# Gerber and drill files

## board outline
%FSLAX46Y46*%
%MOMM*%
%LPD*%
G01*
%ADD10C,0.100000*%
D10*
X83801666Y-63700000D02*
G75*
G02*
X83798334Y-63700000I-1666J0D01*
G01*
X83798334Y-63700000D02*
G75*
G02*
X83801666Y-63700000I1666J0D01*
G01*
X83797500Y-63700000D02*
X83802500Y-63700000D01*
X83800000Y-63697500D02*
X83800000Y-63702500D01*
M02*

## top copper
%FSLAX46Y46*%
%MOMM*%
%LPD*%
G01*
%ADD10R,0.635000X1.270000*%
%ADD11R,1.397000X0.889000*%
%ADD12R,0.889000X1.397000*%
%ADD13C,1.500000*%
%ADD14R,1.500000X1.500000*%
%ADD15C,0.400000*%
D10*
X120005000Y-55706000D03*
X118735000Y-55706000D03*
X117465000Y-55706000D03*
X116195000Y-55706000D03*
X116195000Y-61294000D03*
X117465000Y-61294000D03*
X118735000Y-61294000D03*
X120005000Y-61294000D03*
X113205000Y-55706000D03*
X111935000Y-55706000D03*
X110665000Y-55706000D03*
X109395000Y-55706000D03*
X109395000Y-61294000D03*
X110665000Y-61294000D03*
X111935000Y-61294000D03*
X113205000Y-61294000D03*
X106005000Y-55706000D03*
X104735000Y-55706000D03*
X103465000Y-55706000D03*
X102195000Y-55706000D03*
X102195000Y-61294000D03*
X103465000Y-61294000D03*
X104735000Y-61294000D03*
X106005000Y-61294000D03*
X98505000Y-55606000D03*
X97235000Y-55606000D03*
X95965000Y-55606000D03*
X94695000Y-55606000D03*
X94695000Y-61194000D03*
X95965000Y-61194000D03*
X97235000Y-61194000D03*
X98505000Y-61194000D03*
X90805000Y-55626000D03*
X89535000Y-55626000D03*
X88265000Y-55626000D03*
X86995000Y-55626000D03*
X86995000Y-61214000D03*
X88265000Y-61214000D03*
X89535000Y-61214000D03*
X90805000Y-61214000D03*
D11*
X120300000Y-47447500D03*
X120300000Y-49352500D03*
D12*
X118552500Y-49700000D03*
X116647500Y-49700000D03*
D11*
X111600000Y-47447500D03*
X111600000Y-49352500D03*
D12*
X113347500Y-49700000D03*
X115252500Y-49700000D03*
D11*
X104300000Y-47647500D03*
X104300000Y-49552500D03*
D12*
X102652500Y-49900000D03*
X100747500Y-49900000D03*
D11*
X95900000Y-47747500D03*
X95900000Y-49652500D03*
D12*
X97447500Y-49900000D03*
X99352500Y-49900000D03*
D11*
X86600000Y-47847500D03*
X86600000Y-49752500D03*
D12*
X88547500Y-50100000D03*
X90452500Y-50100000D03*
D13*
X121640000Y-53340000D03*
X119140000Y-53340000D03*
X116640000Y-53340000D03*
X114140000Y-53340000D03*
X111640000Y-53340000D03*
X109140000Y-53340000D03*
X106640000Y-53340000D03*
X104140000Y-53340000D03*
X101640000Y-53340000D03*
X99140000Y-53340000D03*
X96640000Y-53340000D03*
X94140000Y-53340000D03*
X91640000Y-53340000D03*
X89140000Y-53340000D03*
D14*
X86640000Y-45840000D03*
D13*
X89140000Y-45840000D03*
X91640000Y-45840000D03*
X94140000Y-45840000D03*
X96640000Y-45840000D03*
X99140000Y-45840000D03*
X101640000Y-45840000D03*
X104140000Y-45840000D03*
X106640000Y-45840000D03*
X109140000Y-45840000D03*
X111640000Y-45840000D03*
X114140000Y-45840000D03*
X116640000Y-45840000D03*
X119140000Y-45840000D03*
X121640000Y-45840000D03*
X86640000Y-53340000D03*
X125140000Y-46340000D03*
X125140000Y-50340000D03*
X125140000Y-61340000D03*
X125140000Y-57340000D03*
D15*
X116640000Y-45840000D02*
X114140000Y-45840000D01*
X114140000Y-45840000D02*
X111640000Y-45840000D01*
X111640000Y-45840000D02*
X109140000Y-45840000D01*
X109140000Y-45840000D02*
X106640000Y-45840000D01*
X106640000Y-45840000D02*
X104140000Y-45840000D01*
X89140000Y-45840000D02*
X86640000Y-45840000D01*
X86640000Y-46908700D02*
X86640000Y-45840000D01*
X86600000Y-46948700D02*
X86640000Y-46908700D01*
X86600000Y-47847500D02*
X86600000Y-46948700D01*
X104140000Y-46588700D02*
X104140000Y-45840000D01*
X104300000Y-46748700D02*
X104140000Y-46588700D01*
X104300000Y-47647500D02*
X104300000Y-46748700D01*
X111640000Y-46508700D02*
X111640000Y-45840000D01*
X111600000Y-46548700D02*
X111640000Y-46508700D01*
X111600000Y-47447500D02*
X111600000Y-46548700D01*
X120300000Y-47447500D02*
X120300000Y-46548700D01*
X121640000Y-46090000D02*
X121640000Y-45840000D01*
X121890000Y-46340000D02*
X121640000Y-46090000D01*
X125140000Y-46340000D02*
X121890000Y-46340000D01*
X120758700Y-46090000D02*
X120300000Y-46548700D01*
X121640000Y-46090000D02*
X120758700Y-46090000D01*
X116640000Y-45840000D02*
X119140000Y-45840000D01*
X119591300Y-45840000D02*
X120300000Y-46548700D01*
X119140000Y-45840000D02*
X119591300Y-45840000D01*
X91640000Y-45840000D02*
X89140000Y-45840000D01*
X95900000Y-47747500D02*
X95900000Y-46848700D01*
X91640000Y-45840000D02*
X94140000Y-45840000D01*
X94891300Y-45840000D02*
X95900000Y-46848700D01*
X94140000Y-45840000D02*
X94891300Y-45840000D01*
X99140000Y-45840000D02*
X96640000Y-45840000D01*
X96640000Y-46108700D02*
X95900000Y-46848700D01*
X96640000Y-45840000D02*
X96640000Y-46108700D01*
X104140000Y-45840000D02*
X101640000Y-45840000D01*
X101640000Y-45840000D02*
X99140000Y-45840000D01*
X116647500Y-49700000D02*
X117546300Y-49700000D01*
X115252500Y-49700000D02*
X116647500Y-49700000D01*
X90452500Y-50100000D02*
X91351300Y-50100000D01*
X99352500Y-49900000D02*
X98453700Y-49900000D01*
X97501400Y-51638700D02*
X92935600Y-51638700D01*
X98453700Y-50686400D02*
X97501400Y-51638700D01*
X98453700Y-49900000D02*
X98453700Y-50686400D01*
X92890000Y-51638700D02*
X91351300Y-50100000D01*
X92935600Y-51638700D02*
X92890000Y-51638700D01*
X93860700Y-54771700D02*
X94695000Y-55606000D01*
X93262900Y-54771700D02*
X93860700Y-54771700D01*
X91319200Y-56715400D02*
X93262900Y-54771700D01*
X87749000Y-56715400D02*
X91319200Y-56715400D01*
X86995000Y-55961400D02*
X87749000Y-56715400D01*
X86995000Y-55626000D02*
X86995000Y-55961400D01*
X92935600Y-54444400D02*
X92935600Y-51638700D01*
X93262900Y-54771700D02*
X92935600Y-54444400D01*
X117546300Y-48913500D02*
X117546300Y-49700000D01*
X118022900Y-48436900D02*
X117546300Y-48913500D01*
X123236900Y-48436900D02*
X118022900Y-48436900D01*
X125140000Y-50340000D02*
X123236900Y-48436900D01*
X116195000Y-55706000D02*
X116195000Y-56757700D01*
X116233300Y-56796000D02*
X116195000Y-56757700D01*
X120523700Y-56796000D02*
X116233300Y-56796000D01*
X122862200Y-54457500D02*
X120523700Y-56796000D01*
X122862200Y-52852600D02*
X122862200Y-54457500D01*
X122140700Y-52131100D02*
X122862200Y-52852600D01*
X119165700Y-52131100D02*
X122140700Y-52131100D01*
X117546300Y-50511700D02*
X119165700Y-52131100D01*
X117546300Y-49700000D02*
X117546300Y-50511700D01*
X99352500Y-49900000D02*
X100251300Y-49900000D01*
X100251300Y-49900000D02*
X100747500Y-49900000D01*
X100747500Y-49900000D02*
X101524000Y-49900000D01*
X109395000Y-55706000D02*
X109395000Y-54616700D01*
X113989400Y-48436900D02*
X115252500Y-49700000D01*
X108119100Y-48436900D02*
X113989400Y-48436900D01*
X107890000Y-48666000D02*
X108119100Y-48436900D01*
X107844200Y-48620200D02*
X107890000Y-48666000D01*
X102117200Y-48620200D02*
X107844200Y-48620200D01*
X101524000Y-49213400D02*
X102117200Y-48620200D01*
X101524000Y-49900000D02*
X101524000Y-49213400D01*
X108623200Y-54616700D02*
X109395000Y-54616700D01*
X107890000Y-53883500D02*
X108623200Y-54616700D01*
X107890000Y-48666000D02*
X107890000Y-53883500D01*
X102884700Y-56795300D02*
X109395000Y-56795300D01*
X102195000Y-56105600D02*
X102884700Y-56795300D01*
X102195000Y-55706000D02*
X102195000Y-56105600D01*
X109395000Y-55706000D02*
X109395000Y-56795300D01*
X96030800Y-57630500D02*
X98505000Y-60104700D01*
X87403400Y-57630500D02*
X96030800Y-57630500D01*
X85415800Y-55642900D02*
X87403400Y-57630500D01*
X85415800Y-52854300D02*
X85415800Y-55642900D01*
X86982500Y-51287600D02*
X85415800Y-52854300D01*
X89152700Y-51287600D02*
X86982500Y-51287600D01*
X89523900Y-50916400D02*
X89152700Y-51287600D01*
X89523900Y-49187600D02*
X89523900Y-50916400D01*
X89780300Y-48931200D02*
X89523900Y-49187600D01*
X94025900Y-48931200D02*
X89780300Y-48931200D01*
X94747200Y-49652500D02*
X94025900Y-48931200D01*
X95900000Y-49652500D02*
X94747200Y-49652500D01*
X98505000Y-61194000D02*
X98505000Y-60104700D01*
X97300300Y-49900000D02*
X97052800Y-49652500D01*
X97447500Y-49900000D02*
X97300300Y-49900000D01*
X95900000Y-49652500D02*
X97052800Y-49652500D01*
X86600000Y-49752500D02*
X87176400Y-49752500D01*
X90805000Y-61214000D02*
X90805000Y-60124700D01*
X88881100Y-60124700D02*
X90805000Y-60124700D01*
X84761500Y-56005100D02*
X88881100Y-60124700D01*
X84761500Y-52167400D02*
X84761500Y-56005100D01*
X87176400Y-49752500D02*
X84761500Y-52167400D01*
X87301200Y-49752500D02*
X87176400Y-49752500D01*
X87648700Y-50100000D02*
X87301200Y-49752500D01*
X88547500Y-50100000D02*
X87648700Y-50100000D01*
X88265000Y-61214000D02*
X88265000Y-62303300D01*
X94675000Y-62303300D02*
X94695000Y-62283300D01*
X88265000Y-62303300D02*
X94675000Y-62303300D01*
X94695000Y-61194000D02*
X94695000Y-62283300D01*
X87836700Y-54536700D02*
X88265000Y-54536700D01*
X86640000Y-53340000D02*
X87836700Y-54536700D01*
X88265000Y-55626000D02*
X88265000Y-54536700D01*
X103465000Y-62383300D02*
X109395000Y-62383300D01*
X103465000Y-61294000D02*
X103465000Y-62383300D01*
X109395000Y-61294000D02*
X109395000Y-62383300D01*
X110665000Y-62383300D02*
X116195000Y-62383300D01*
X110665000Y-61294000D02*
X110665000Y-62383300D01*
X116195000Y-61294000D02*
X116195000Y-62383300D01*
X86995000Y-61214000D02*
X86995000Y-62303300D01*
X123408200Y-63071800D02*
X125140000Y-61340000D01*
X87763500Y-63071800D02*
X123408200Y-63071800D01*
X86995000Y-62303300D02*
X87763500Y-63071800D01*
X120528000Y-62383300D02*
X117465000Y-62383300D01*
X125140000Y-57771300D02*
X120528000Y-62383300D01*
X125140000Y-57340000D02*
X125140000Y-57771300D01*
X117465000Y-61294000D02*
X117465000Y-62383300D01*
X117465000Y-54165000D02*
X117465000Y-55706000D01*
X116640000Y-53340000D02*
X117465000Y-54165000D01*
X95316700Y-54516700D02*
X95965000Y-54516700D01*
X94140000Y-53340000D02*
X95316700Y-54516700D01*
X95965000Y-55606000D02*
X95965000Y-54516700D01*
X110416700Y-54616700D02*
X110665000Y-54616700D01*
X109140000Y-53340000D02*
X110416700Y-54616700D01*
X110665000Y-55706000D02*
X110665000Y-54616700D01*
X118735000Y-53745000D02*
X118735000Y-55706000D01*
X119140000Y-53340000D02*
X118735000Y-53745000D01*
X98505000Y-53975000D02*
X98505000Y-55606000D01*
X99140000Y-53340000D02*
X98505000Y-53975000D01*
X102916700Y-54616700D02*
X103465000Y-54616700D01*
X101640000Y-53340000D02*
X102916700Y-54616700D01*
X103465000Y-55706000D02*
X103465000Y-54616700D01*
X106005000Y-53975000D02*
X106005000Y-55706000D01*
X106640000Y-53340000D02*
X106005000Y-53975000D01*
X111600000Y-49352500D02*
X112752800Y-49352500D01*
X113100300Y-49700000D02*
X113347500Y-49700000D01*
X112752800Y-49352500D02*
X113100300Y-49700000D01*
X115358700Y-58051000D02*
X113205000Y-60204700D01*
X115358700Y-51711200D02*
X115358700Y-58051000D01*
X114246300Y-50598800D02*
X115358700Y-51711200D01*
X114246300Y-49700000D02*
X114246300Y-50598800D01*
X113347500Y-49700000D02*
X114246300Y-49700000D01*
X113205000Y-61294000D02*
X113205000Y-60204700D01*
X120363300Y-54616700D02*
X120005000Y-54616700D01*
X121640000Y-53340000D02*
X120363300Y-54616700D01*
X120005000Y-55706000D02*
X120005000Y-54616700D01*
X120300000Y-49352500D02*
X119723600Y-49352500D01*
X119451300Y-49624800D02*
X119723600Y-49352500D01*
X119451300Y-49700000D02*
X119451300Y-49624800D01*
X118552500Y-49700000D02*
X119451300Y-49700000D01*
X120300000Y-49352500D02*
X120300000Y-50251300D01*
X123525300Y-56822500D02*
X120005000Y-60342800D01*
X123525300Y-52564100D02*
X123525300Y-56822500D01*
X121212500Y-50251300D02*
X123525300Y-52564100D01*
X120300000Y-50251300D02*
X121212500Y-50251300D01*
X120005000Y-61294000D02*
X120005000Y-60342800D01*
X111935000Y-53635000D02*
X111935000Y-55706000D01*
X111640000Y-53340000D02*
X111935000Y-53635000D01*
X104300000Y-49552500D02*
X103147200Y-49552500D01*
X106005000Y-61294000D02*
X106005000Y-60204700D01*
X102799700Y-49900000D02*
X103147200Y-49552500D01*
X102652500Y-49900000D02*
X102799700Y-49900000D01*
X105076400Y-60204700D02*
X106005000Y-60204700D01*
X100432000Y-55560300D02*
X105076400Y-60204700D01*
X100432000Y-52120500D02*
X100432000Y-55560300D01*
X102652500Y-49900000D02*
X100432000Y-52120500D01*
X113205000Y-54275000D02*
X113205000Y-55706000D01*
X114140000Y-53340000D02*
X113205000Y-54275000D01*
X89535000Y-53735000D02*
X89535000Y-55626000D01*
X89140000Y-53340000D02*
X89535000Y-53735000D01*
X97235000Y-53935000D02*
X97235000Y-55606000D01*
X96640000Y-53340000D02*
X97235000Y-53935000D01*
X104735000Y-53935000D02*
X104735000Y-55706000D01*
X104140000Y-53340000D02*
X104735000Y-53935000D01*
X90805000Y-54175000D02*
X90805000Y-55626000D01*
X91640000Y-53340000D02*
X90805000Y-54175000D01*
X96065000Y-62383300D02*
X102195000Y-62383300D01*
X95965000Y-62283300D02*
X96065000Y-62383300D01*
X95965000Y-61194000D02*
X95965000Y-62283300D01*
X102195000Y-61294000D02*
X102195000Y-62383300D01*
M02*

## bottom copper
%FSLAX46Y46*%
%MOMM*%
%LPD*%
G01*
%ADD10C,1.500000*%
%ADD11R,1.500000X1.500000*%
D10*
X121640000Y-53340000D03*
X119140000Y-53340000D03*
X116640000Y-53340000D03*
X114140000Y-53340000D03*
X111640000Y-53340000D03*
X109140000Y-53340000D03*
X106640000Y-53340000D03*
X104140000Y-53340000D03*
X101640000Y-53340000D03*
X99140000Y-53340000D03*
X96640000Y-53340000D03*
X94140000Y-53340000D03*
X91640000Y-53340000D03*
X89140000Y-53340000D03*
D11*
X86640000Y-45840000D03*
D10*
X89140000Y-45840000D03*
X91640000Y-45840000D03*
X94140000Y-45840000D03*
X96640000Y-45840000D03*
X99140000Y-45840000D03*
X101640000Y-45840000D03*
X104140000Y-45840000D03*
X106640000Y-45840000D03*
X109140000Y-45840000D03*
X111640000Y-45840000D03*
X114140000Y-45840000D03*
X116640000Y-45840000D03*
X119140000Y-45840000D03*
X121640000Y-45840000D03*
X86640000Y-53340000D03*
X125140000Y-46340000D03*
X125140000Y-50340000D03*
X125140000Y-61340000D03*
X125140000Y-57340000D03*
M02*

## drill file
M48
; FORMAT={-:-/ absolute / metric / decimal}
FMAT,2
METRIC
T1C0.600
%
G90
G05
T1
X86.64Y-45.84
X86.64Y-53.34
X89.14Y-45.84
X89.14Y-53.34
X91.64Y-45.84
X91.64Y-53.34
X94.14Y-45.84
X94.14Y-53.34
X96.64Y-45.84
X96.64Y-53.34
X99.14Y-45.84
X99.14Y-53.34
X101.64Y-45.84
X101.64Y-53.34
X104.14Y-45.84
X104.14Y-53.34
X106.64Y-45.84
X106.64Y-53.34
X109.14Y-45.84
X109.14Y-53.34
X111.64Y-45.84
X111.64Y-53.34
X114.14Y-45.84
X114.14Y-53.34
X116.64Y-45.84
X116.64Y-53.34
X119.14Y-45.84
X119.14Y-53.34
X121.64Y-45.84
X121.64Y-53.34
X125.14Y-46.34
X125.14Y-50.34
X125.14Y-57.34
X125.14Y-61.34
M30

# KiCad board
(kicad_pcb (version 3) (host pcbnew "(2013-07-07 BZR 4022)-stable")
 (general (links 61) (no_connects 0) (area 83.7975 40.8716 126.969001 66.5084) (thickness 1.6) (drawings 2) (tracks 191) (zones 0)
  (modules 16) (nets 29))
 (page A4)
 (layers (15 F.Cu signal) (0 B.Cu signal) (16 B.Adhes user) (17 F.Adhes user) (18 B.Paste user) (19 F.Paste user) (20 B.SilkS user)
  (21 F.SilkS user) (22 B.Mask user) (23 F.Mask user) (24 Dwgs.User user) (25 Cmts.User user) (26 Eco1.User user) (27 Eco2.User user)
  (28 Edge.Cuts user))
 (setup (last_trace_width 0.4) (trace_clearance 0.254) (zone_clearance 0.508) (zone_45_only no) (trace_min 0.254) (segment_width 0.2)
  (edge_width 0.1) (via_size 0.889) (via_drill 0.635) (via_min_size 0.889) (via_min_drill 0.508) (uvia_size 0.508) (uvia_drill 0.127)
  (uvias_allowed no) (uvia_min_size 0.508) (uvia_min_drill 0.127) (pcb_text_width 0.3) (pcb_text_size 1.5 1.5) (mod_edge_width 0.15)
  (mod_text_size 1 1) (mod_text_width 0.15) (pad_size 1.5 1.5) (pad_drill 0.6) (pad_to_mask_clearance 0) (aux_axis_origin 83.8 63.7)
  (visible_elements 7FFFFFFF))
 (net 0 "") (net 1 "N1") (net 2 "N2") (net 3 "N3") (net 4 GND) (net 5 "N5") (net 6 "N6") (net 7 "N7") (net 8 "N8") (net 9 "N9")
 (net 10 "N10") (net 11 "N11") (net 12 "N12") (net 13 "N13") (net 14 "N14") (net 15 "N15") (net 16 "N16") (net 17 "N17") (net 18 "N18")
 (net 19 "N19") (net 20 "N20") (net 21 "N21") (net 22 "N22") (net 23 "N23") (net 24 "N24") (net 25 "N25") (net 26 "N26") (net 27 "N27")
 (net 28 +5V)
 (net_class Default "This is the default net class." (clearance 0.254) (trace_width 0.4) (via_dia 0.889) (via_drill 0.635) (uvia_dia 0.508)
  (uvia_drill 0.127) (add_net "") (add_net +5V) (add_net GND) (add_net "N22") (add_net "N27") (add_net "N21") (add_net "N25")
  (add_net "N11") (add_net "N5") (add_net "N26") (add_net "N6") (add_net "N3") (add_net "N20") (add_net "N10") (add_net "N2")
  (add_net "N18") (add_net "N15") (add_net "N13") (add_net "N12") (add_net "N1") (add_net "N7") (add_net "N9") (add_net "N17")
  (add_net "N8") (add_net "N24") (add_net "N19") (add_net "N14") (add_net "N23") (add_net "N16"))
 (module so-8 (layer F.Cu) (at 118.1 58.5 180)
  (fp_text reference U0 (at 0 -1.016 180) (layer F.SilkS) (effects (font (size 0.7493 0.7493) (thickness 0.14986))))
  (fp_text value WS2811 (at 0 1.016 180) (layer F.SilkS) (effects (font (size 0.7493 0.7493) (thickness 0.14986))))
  (pad 1 smd rect (at -1.905 2.794 180) (size 0.635 1.27) (layers F.Cu F.Paste F.Mask) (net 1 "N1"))
  (pad 2 smd rect (at -0.635 2.794 180) (size 0.635 1.27) (layers F.Cu F.Paste F.Mask) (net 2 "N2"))
  (pad 3 smd rect (at 0.635 2.794 180) (size 0.635 1.27) (layers F.Cu F.Paste F.Mask) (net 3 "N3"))
  (pad 4 smd rect (at 1.905 2.794 180) (size 0.635 1.27) (layers F.Cu F.Paste F.Mask) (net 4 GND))
  (pad 5 smd rect (at 1.905 -2.794 180) (size 0.635 1.27) (layers F.Cu F.Paste F.Mask) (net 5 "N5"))
  (pad 6 smd rect (at 0.635 -2.794 180) (size 0.635 1.27) (layers F.Cu F.Paste F.Mask) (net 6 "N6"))
  (pad 7 smd rect (at -0.635 -2.794 180) (size 0.635 1.27) (layers F.Cu F.Paste F.Mask))
  (pad 8 smd rect (at -1.905 -2.794 180) (size 0.635 1.27) (layers F.Cu F.Paste F.Mask) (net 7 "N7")))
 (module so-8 (layer F.Cu) (at 111.3 58.5 180)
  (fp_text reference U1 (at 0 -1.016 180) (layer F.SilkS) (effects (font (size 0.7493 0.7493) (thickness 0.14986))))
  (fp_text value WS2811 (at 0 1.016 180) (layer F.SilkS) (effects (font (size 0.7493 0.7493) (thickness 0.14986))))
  (pad 1 smd rect (at -1.905 2.794 180) (size 0.635 1.27) (layers F.Cu F.Paste F.Mask) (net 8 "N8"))
  (pad 2 smd rect (at -0.635 2.794 180) (size 0.635 1.27) (layers F.Cu F.Paste F.Mask) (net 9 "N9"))
  (pad 3 smd rect (at 0.635 2.794 180) (size 0.635 1.27) (layers F.Cu F.Paste F.Mask) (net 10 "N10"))
  (pad 4 smd rect (at 1.905 2.794 180) (size 0.635 1.27) (layers F.Cu F.Paste F.Mask) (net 4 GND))
  (pad 5 smd rect (at 1.905 -2.794 180) (size 0.635 1.27) (layers F.Cu F.Paste F.Mask) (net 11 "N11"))
  (pad 6 smd rect (at 0.635 -2.794 180) (size 0.635 1.27) (layers F.Cu F.Paste F.Mask) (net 5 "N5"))
  (pad 7 smd rect (at -0.635 -2.794 180) (size 0.635 1.27) (layers F.Cu F.Paste F.Mask))
  (pad 8 smd rect (at -1.905 -2.794 180) (size 0.635 1.27) (layers F.Cu F.Paste F.Mask) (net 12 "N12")))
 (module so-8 (layer F.Cu) (at 104.1 58.5 180)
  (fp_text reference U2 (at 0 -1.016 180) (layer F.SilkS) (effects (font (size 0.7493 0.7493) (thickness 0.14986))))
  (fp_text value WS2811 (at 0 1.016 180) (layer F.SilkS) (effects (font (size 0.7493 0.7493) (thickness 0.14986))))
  (pad 1 smd rect (at -1.905 2.794 180) (size 0.635 1.27) (layers F.Cu F.Paste F.Mask) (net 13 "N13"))
  (pad 2 smd rect (at -0.635 2.794 180) (size 0.635 1.27) (layers F.Cu F.Paste F.Mask) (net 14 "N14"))
  (pad 3 smd rect (at 0.635 2.794 180) (size 0.635 1.27) (layers F.Cu F.Paste F.Mask) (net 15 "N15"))
  (pad 4 smd rect (at 1.905 2.794 180) (size 0.635 1.27) (layers F.Cu F.Paste F.Mask) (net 4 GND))
  (pad 5 smd rect (at 1.905 -2.794 180) (size 0.635 1.27) (layers F.Cu F.Paste F.Mask) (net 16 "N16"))
  (pad 6 smd rect (at 0.635 -2.794 180) (size 0.635 1.27) (layers F.Cu F.Paste F.Mask) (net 11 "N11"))
  (pad 7 smd rect (at -0.635 -2.794 180) (size 0.635 1.27) (layers F.Cu F.Paste F.Mask))
  (pad 8 smd rect (at -1.905 -2.794 180) (size 0.635 1.27) (layers F.Cu F.Paste F.Mask) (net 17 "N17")))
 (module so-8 (layer F.Cu) (at 96.6 58.4 180)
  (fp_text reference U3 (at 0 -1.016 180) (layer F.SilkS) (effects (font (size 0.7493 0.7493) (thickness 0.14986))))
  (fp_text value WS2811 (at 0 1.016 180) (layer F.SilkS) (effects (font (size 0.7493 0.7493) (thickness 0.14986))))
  (pad 1 smd rect (at -1.905 2.794 180) (size 0.635 1.27) (layers F.Cu F.Paste F.Mask) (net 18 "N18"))
  (pad 2 smd rect (at -0.635 2.794 180) (size 0.635 1.27) (layers F.Cu F.Paste F.Mask) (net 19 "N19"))
  (pad 3 smd rect (at 0.635 2.794 180) (size 0.635 1.27) (layers F.Cu F.Paste F.Mask) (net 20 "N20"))
  (pad 4 smd rect (at 1.905 2.794 180) (size 0.635 1.27) (layers F.Cu F.Paste F.Mask) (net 4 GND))
  (pad 5 smd rect (at 1.905 -2.794 180) (size 0.635 1.27) (layers F.Cu F.Paste F.Mask) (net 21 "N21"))
  (pad 6 smd rect (at 0.635 -2.794 180) (size 0.635 1.27) (layers F.Cu F.Paste F.Mask) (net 16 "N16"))
  (pad 7 smd rect (at -0.635 -2.794 180) (size 0.635 1.27) (layers F.Cu F.Paste F.Mask))
  (pad 8 smd rect (at -1.905 -2.794 180) (size 0.635 1.27) (layers F.Cu F.Paste F.Mask) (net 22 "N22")))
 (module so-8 (layer F.Cu) (at 88.9 58.42 180)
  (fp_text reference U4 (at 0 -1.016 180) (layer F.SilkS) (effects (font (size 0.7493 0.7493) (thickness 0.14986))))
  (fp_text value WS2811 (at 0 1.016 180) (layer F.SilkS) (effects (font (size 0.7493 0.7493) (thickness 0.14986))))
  (pad 1 smd rect (at -1.905 2.794 180) (size 0.635 1.27) (layers F.Cu F.Paste F.Mask) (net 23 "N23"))
  (pad 2 smd rect (at -0.635 2.794 180) (size 0.635 1.27) (layers F.Cu F.Paste F.Mask) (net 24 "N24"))
  (pad 3 smd rect (at 0.635 2.794 180) (size 0.635 1.27) (layers F.Cu F.Paste F.Mask) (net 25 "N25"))
  (pad 4 smd rect (at 1.905 2.794 180) (size 0.635 1.27) (layers F.Cu F.Paste F.Mask) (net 4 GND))
  (pad 5 smd rect (at 1.905 -2.794 180) (size 0.635 1.27) (layers F.Cu F.Paste F.Mask) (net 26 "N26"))
  (pad 6 smd rect (at 0.635 -2.794 180) (size 0.635 1.27) (layers F.Cu F.Paste F.Mask) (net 21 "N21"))
  (pad 7 smd rect (at -0.635 -2.794 180) (size 0.635 1.27) (layers F.Cu F.Paste F.Mask))
  (pad 8 smd rect (at -1.905 -2.794 180) (size 0.635 1.27) (layers F.Cu F.Paste F.Mask) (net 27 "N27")))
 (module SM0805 (layer F.Cu) (at 120.3 48.4 270)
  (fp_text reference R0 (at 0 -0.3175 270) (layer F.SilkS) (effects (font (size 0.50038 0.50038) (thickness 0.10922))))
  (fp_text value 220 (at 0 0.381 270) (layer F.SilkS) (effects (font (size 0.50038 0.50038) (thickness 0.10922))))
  (pad 1 smd rect (at -0.9525 0 270) (size 0.889 1.397) (layers F.Cu F.Paste F.Mask) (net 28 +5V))
  (pad 2 smd rect (at 0.9525 0 270) (size 0.889 1.397) (layers F.Cu F.Paste F.Mask) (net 7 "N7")))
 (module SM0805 (layer F.Cu) (at 117.6 49.7 180)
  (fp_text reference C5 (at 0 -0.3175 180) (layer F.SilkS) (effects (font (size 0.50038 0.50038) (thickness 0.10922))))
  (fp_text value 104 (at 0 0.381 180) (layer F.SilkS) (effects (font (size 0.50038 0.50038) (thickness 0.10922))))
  (pad 1 smd rect (at -0.9525 0 180) (size 0.889 1.397) (layers F.Cu F.Paste F.Mask) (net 7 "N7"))
  (pad 2 smd rect (at 0.9525 0 180) (size 0.889 1.397) (layers F.Cu F.Paste F.Mask) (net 4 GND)))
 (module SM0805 (layer F.Cu) (at 111.6 48.4 270)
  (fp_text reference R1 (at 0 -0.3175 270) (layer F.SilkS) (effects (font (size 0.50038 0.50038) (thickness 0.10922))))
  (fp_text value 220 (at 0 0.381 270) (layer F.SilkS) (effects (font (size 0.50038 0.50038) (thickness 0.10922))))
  (pad 1 smd rect (at -0.9525 0 270) (size 0.889 1.397) (layers F.Cu F.Paste F.Mask) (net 28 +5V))
  (pad 2 smd rect (at 0.9525 0 270) (size 0.889 1.397) (layers F.Cu F.Paste F.Mask) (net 12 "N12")))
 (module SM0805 (layer F.Cu) (at 114.3 49.7)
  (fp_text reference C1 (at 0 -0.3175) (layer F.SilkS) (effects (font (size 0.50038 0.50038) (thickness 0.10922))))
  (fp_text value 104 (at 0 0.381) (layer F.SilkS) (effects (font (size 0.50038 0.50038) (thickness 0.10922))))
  (pad 1 smd rect (at -0.9525 0) (size 0.889 1.397) (layers F.Cu F.Paste F.Mask) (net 12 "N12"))
  (pad 2 smd rect (at 0.9525 0) (size 0.889 1.397) (layers F.Cu F.Paste F.Mask) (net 4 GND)))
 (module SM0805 (layer F.Cu) (at 104.3 48.6 270)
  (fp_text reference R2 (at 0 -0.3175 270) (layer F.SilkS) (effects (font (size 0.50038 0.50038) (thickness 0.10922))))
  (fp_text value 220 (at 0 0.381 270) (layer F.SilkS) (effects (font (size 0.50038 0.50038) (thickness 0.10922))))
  (pad 1 smd rect (at -0.9525 0 270) (size 0.889 1.397) (layers F.Cu F.Paste F.Mask) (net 28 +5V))
  (pad 2 smd rect (at 0.9525 0 270) (size 0.889 1.397) (layers F.Cu F.Paste F.Mask) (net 17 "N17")))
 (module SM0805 (layer F.Cu) (at 101.7 49.9 180)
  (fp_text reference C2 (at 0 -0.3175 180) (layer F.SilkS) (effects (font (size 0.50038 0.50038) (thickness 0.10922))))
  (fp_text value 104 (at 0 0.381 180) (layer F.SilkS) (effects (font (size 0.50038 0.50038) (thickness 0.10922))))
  (pad 1 smd rect (at -0.9525 0 180) (size 0.889 1.397) (layers F.Cu F.Paste F.Mask) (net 17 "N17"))
  (pad 2 smd rect (at 0.9525 0 180) (size 0.889 1.397) (layers F.Cu F.Paste F.Mask) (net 4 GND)))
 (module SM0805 (layer F.Cu) (at 95.9 48.7 270)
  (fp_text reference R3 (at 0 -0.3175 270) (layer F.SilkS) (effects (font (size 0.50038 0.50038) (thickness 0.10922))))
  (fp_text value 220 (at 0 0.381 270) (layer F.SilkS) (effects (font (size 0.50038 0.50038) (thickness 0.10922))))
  (pad 1 smd rect (at -0.9525 0 270) (size 0.889 1.397) (layers F.Cu F.Paste F.Mask) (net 28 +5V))
  (pad 2 smd rect (at 0.9525 0 270) (size 0.889 1.397) (layers F.Cu F.Paste F.Mask) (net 22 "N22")))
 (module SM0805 (layer F.Cu) (at 98.4 49.9)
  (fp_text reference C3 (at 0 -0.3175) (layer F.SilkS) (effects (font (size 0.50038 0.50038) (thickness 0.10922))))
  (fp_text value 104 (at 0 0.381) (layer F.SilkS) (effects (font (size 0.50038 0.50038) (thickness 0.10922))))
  (pad 1 smd rect (at -0.9525 0) (size 0.889 1.397) (layers F.Cu F.Paste F.Mask) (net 22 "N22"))
  (pad 2 smd rect (at 0.9525 0) (size 0.889 1.397) (layers F.Cu F.Paste F.Mask) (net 4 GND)))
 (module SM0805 (layer F.Cu) (at 86.6 48.8 270)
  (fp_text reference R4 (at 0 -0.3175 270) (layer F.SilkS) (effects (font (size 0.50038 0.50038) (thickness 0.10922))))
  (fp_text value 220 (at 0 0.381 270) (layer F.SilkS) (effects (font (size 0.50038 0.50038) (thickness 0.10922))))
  (pad 1 smd rect (at -0.9525 0 270) (size 0.889 1.397) (layers F.Cu F.Paste F.Mask) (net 28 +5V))
  (pad 2 smd rect (at 0.9525 0 270) (size 0.889 1.397) (layers F.Cu F.Paste F.Mask) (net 27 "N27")))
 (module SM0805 (layer F.Cu) (at 89.5 50.1)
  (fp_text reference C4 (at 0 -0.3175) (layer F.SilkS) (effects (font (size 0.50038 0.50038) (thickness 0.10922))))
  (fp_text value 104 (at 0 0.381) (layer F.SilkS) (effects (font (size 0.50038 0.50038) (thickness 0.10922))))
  (pad 1 smd rect (at -0.9525 0) (size 0.889 1.397) (layers F.Cu F.Paste F.Mask) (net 27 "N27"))
  (pad 2 smd rect (at 0.9525 0) (size 0.889 1.397) (layers F.Cu F.Paste F.Mask) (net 4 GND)))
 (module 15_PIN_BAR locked (layer F.Cu) (at 104.14 53.34)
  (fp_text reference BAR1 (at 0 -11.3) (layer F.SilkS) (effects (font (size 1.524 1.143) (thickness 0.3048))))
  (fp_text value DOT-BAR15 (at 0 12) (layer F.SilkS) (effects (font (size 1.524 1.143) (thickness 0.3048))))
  (pad 16 thru_hole circle (at 17.5 0) (size 1.5 1.5) (drill 0.6) (layers *.Cu *.Mask F.SilkS) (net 1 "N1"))
  (pad 17 thru_hole circle (at 15 0) (size 1.5 1.5) (drill 0.6) (layers *.Cu *.Mask F.SilkS) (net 2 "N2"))
  (pad 18 thru_hole circle (at 12.5 0) (size 1.5 1.5) (drill 0.6) (layers *.Cu *.Mask F.SilkS) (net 3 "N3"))
  (pad 19 thru_hole circle (at 10 0) (size 1.5 1.5) (drill 0.6) (layers *.Cu *.Mask F.SilkS) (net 8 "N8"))
  (pad 20 thru_hole circle (at 7.5 0) (size 1.5 1.5) (drill 0.6) (layers *.Cu *.Mask F.SilkS) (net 9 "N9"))
  (pad 21 thru_hole circle (at 5 0) (size 1.5 1.5) (drill 0.6) (layers *.Cu *.Mask F.SilkS) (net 10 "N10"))
  (pad 22 thru_hole circle (at 2.5 0) (size 1.5 1.5) (drill 0.6) (layers *.Cu *.Mask F.SilkS) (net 13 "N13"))
  (pad 23 thru_hole circle (at 0 0) (size 1.5 1.5) (drill 0.6) (layers *.Cu *.Mask F.SilkS) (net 14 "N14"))
  (pad 24 thru_hole circle (at -2.5 0) (size 1.5 1.5) (drill 0.6) (layers *.Cu *.Mask F.SilkS) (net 15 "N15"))
  (pad 25 thru_hole circle (at -5 0) (size 1.5 1.5) (drill 0.6) (layers *.Cu *.Mask F.SilkS) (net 18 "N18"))
  (pad 26 thru_hole circle (at -7.5 0) (size 1.5 1.5) (drill 0.6) (layers *.Cu *.Mask F.SilkS) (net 19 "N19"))
  (pad 27 thru_hole circle (at -10 0) (size 1.5 1.5) (drill 0.6) (layers *.Cu *.Mask F.SilkS) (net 20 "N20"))
  (pad 28 thru_hole circle (at -12.5 0) (size 1.5 1.5) (drill 0.6) (layers *.Cu *.Mask F.SilkS) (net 23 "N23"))
  (pad 29 thru_hole circle (at -15 0) (size 1.5 1.5) (drill 0.6) (layers *.Cu *.Mask F.SilkS) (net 24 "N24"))
  (pad 1 thru_hole rect (at -17.5 -7.5) (size 1.5 1.5) (drill 0.6) (layers *.Cu *.Mask F.SilkS) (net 28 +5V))
  (pad 2 thru_hole circle (at -15 -7.5) (size 1.5 1.5) (drill 0.6) (layers *.Cu *.Mask F.SilkS) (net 28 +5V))
  (pad 3 thru_hole circle (at -12.5 -7.5) (size 1.5 1.5) (drill 0.6) (layers *.Cu *.Mask F.SilkS) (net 28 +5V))
  (pad 4 thru_hole circle (at -10 -7.5) (size 1.5 1.5) (drill 0.6) (layers *.Cu *.Mask F.SilkS) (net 28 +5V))
  (pad 5 thru_hole circle (at -7.5 -7.5) (size 1.5 1.5) (drill 0.6) (layers *.Cu *.Mask F.SilkS) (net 28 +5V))
  (pad 6 thru_hole circle (at -5 -7.5) (size 1.5 1.5) (drill 0.6) (layers *.Cu *.Mask F.SilkS) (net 28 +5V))
  (pad 7 thru_hole circle (at -2.5 -7.5) (size 1.5 1.5) (drill 0.6) (layers *.Cu *.Mask F.SilkS) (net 28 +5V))
  (pad 8 thru_hole circle (at 0 -7.5) (size 1.5 1.5) (drill 0.6) (layers *.Cu *.Mask F.SilkS) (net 28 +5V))
  (pad 9 thru_hole circle (at 2.5 -7.5) (size 1.5 1.5) (drill 0.6) (layers *.Cu *.Mask F.SilkS) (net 28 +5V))
  (pad 10 thru_hole circle (at 5 -7.5) (size 1.5 1.5) (drill 0.6) (layers *.Cu *.Mask F.SilkS) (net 28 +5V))
  (pad 11 thru_hole circle (at 7.5 -7.5) (size 1.5 1.5) (drill 0.6) (layers *.Cu *.Mask F.SilkS) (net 28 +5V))
  (pad 12 thru_hole circle (at 10 -7.5) (size 1.5 1.5) (drill 0.6) (layers *.Cu *.Mask F.SilkS) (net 28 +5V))
  (pad 13 thru_hole circle (at 12.5 -7.5) (size 1.5 1.5) (drill 0.6) (layers *.Cu *.Mask F.SilkS) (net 28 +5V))
  (pad 14 thru_hole circle (at 15 -7.5) (size 1.5 1.5) (drill 0.6) (layers *.Cu *.Mask F.SilkS) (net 28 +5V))
  (pad 15 thru_hole circle (at 17.5 -7.5) (size 1.5 1.5) (drill 0.6) (layers *.Cu *.Mask F.SilkS) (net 28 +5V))
  (pad 30 thru_hole circle (at -17.5 0) (size 1.5 1.5) (drill 0.6) (layers *.Cu *.Mask F.SilkS) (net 25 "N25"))
  (pad 31 thru_hole circle (at 21 -7) (size 1.5 1.5) (drill 0.6) (layers *.Cu *.Mask F.SilkS) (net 28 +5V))
  (pad 32 thru_hole circle (at 21 -3) (size 1.5 1.5) (drill 0.6) (layers *.Cu *.Mask F.SilkS) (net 4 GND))
  (pad 33 thru_hole circle (at 21 8) (size 1.5 1.5) (drill 0.6) (layers *.Cu *.Mask F.SilkS) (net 26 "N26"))
  (pad 34 thru_hole circle (at 21 4) (size 1.5 1.5) (drill 0.6) (layers *.Cu *.Mask F.SilkS) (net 6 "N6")))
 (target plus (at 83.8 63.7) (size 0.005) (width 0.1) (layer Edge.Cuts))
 (segment (start 116.64 45.84) (end 114.14 45.84) (width 0.4) (layer F.Cu) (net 28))
 (segment (start 114.14 45.84) (end 111.64 45.84) (width 0.4) (layer F.Cu) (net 28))
 (segment (start 111.64 45.84) (end 109.14 45.84) (width 0.4) (layer F.Cu) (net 28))
 (segment (start 109.14 45.84) (end 106.64 45.84) (width 0.4) (layer F.Cu) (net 28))
 (segment (start 106.64 45.84) (end 104.14 45.84) (width 0.4) (layer F.Cu) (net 28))
 (segment (start 89.14 45.84) (end 86.64 45.84) (width 0.4) (layer F.Cu) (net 28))
 (segment (start 86.64 46.9087) (end 86.64 45.84) (width 0.4) (layer F.Cu) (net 28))
 (segment (start 86.6 46.9487) (end 86.64 46.9087) (width 0.4) (layer F.Cu) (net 28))
 (segment (start 86.6 47.8475) (end 86.6 46.9487) (width 0.4) (layer F.Cu) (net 28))
 (segment (start 104.14 46.5887) (end 104.14 45.84) (width 0.4) (layer F.Cu) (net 28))
 (segment (start 104.3 46.7487) (end 104.14 46.5887) (width 0.4) (layer F.Cu) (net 28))
 (segment (start 104.3 47.6475) (end 104.3 46.7487) (width 0.4) (layer F.Cu) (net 28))
 (segment (start 111.64 46.5087) (end 111.64 45.84) (width 0.4) (layer F.Cu) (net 28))
 (segment (start 111.6 46.5487) (end 111.64 46.5087) (width 0.4) (layer F.Cu) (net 28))
 (segment (start 111.6 47.4475) (end 111.6 46.5487) (width 0.4) (layer F.Cu) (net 28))
 (segment (start 120.3 47.4475) (end 120.3 46.5487) (width 0.4) (layer F.Cu) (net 28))
 (segment (start 121.64 46.09) (end 121.64 45.84) (width 0.4) (layer F.Cu) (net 28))
 (segment (start 121.89 46.34) (end 121.64 46.09) (width 0.4) (layer F.Cu) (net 28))
 (segment (start 125.14 46.34) (end 121.89 46.34) (width 0.4) (layer F.Cu) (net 28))
 (segment (start 120.7587 46.09) (end 120.3 46.5487) (width 0.4) (layer F.Cu) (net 28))
 (segment (start 121.64 46.09) (end 120.7587 46.09) (width 0.4) (layer F.Cu) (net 28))
 (segment (start 116.64 45.84) (end 119.14 45.84) (width 0.4) (layer F.Cu) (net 28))
 (segment (start 119.5913 45.84) (end 120.3 46.5487) (width 0.4) (layer F.Cu) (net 28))
 (segment (start 119.14 45.84) (end 119.5913 45.84) (width 0.4) (layer F.Cu) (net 28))
 (segment (start 91.64 45.84) (end 89.14 45.84) (width 0.4) (layer F.Cu) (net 28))
 (segment (start 95.9 47.7475) (end 95.9 46.8487) (width 0.4) (layer F.Cu) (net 28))
 (segment (start 91.64 45.84) (end 94.14 45.84) (width 0.4) (layer F.Cu) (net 28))
 (segment (start 94.8913 45.84) (end 95.9 46.8487) (width 0.4) (layer F.Cu) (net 28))
 (segment (start 94.14 45.84) (end 94.8913 45.84) (width 0.4) (layer F.Cu) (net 28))
 (segment (start 99.14 45.84) (end 96.64 45.84) (width 0.4) (layer F.Cu) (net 28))
 (segment (start 96.64 46.1087) (end 95.9 46.8487) (width 0.4) (layer F.Cu) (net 28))
 (segment (start 96.64 45.84) (end 96.64 46.1087) (width 0.4) (layer F.Cu) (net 28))
 (segment (start 104.14 45.84) (end 101.64 45.84) (width 0.4) (layer F.Cu) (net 28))
 (segment (start 101.64 45.84) (end 99.14 45.84) (width 0.4) (layer F.Cu) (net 28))
 (segment (start 116.6475 49.7) (end 117.5463 49.7) (width 0.4) (layer F.Cu) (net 4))
 (segment (start 115.2525 49.7) (end 116.6475 49.7) (width 0.4) (layer F.Cu) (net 4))
 (segment (start 90.4525 50.1) (end 91.3513 50.1) (width 0.4) (layer F.Cu) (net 4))
 (segment (start 99.3525 49.9) (end 98.4537 49.9) (width 0.4) (layer F.Cu) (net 4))
 (segment (start 97.5014 51.6387) (end 92.9356 51.6387) (width 0.4) (layer F.Cu) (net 4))
 (segment (start 98.4537 50.6864) (end 97.5014 51.6387) (width 0.4) (layer F.Cu) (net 4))
 (segment (start 98.4537 49.9) (end 98.4537 50.6864) (width 0.4) (layer F.Cu) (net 4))
 (segment (start 92.89 51.6387) (end 91.3513 50.1) (width 0.4) (layer F.Cu) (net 4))
 (segment (start 92.9356 51.6387) (end 92.89 51.6387) (width 0.4) (layer F.Cu) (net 4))
 (segment (start 93.8607 54.7717) (end 94.695 55.606) (width 0.4) (layer F.Cu) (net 4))
 (segment (start 93.2629 54.7717) (end 93.8607 54.7717) (width 0.4) (layer F.Cu) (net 4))
 (segment (start 91.3192 56.7154) (end 93.2629 54.7717) (width 0.4) (layer F.Cu) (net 4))
 (segment (start 87.749 56.7154) (end 91.3192 56.7154) (width 0.4) (layer F.Cu) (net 4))
 (segment (start 86.995 55.9614) (end 87.749 56.7154) (width 0.4) (layer F.Cu) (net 4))
 (segment (start 86.995 55.626) (end 86.995 55.9614) (width 0.4) (layer F.Cu) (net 4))
 (segment (start 92.9356 54.4444) (end 92.9356 51.6387) (width 0.4) (layer F.Cu) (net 4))
 (segment (start 93.2629 54.7717) (end 92.9356 54.4444) (width 0.4) (layer F.Cu) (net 4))
 (segment (start 117.5463 48.9135) (end 117.5463 49.7) (width 0.4) (layer F.Cu) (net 4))
 (segment (start 118.0229 48.4369) (end 117.5463 48.9135) (width 0.4) (layer F.Cu) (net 4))
 (segment (start 123.2369 48.4369) (end 118.0229 48.4369) (width 0.4) (layer F.Cu) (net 4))
 (segment (start 125.14 50.34) (end 123.2369 48.4369) (width 0.4) (layer F.Cu) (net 4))
 (segment (start 116.195 55.706) (end 116.195 56.7577) (width 0.4) (layer F.Cu) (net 4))
 (segment (start 116.2333 56.796) (end 116.195 56.7577) (width 0.4) (layer F.Cu) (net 4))
 (segment (start 120.5237 56.796) (end 116.2333 56.796) (width 0.4) (layer F.Cu) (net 4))
 (segment (start 122.8622 54.4575) (end 120.5237 56.796) (width 0.4) (layer F.Cu) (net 4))
 (segment (start 122.8622 52.8526) (end 122.8622 54.4575) (width 0.4) (layer F.Cu) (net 4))
 (segment (start 122.1407 52.1311) (end 122.8622 52.8526) (width 0.4) (layer F.Cu) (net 4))
 (segment (start 119.1657 52.1311) (end 122.1407 52.1311) (width 0.4) (layer F.Cu) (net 4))
 (segment (start 117.5463 50.5117) (end 119.1657 52.1311) (width 0.4) (layer F.Cu) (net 4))
 (segment (start 117.5463 49.7) (end 117.5463 50.5117) (width 0.4) (layer F.Cu) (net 4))
 (segment (start 99.3525 49.9) (end 100.2513 49.9) (width 0.4) (layer F.Cu) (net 4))
 (segment (start 100.2513 49.9) (end 100.7475 49.9) (width 0.4) (layer F.Cu) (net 4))
 (segment (start 100.7475 49.9) (end 101.524 49.9) (width 0.4) (layer F.Cu) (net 4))
 (segment (start 109.395 55.706) (end 109.395 54.6167) (width 0.4) (layer F.Cu) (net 4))
 (segment (start 113.9894 48.4369) (end 115.2525 49.7) (width 0.4) (layer F.Cu) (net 4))
 (segment (start 108.1191 48.4369) (end 113.9894 48.4369) (width 0.4) (layer F.Cu) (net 4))
 (segment (start 107.89 48.666) (end 108.1191 48.4369) (width 0.4) (layer F.Cu) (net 4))
 (segment (start 107.8442 48.6202) (end 107.89 48.666) (width 0.4) (layer F.Cu) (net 4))
 (segment (start 102.1172 48.6202) (end 107.8442 48.6202) (width 0.4) (layer F.Cu) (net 4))
 (segment (start 101.524 49.2134) (end 102.1172 48.6202) (width 0.4) (layer F.Cu) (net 4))
 (segment (start 101.524 49.9) (end 101.524 49.2134) (width 0.4) (layer F.Cu) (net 4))
 (segment (start 108.6232 54.6167) (end 109.395 54.6167) (width 0.4) (layer F.Cu) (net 4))
 (segment (start 107.89 53.8835) (end 108.6232 54.6167) (width 0.4) (layer F.Cu) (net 4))
 (segment (start 107.89 48.666) (end 107.89 53.8835) (width 0.4) (layer F.Cu) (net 4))
 (segment (start 102.8847 56.7953) (end 109.395 56.7953) (width 0.4) (layer F.Cu) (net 4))
 (segment (start 102.195 56.1056) (end 102.8847 56.7953) (width 0.4) (layer F.Cu) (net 4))
 (segment (start 102.195 55.706) (end 102.195 56.1056) (width 0.4) (layer F.Cu) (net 4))
 (segment (start 109.395 55.706) (end 109.395 56.7953) (width 0.4) (layer F.Cu) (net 4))
 (segment (start 96.0308 57.6305) (end 98.505 60.1047) (width 0.4) (layer F.Cu) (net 22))
 (segment (start 87.4034 57.6305) (end 96.0308 57.6305) (width 0.4) (layer F.Cu) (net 22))
 (segment (start 85.4158 55.6429) (end 87.4034 57.6305) (width 0.4) (layer F.Cu) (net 22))
 (segment (start 85.4158 52.8543) (end 85.4158 55.6429) (width 0.4) (layer F.Cu) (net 22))
 (segment (start 86.9825 51.2876) (end 85.4158 52.8543) (width 0.4) (layer F.Cu) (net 22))
 (segment (start 89.1527 51.2876) (end 86.9825 51.2876) (width 0.4) (layer F.Cu) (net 22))
 (segment (start 89.5239 50.9164) (end 89.1527 51.2876) (width 0.4) (layer F.Cu) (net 22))
 (segment (start 89.5239 49.1876) (end 89.5239 50.9164) (width 0.4) (layer F.Cu) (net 22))
 (segment (start 89.7803 48.9312) (end 89.5239 49.1876) (width 0.4) (layer F.Cu) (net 22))
 (segment (start 94.0259 48.9312) (end 89.7803 48.9312) (width 0.4) (layer F.Cu) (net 22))
 (segment (start 94.7472 49.6525) (end 94.0259 48.9312) (width 0.4) (layer F.Cu) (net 22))
 (segment (start 95.9 49.6525) (end 94.7472 49.6525) (width 0.4) (layer F.Cu) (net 22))
 (segment (start 98.505 61.194) (end 98.505 60.1047) (width 0.4) (layer F.Cu) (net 22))
 (segment (start 97.3003 49.9) (end 97.0528 49.6525) (width 0.4) (layer F.Cu) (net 22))
 (segment (start 97.4475 49.9) (end 97.3003 49.9) (width 0.4) (layer F.Cu) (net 22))
 (segment (start 95.9 49.6525) (end 97.0528 49.6525) (width 0.4) (layer F.Cu) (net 22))
 (segment (start 86.6 49.7525) (end 87.1764 49.7525) (width 0.4) (layer F.Cu) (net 27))
 (segment (start 90.805 61.214) (end 90.805 60.1247) (width 0.4) (layer F.Cu) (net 27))
 (segment (start 88.8811 60.1247) (end 90.805 60.1247) (width 0.4) (layer F.Cu) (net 27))
 (segment (start 84.7615 56.0051) (end 88.8811 60.1247) (width 0.4) (layer F.Cu) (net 27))
 (segment (start 84.7615 52.1674) (end 84.7615 56.0051) (width 0.4) (layer F.Cu) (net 27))
 (segment (start 87.1764 49.7525) (end 84.7615 52.1674) (width 0.4) (layer F.Cu) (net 27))
 (segment (start 87.3012 49.7525) (end 87.1764 49.7525) (width 0.4) (layer F.Cu) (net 27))
 (segment (start 87.6487 50.1) (end 87.3012 49.7525) (width 0.4) (layer F.Cu) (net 27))
 (segment (start 88.5475 50.1) (end 87.6487 50.1) (width 0.4) (layer F.Cu) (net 27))
 (segment (start 88.265 61.214) (end 88.265 62.3033) (width 0.4) (layer F.Cu) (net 21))
 (segment (start 94.675 62.3033) (end 94.695 62.2833) (width 0.4) (layer F.Cu) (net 21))
 (segment (start 88.265 62.3033) (end 94.675 62.3033) (width 0.4) (layer F.Cu) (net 21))
 (segment (start 94.695 61.194) (end 94.695 62.2833) (width 0.4) (layer F.Cu) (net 21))
 (segment (start 87.8367 54.5367) (end 88.265 54.5367) (width 0.4) (layer F.Cu) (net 25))
 (segment (start 86.64 53.34) (end 87.8367 54.5367) (width 0.4) (layer F.Cu) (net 25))
 (segment (start 88.265 55.626) (end 88.265 54.5367) (width 0.4) (layer F.Cu) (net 25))
 (segment (start 103.465 62.3833) (end 109.395 62.3833) (width 0.4) (layer F.Cu) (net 11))
 (segment (start 103.465 61.294) (end 103.465 62.3833) (width 0.4) (layer F.Cu) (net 11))
 (segment (start 109.395 61.294) (end 109.395 62.3833) (width 0.4) (layer F.Cu) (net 11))
 (segment (start 110.665 62.3833) (end 116.195 62.3833) (width 0.4) (layer F.Cu) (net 5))
 (segment (start 110.665 61.294) (end 110.665 62.3833) (width 0.4) (layer F.Cu) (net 5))
 (segment (start 116.195 61.294) (end 116.195 62.3833) (width 0.4) (layer F.Cu) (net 5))
 (segment (start 86.995 61.214) (end 86.995 62.3033) (width 0.4) (layer F.Cu) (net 26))
 (segment (start 123.4082 63.0718) (end 125.14 61.34) (width 0.4) (layer F.Cu) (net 26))
 (segment (start 87.7635 63.0718) (end 123.4082 63.0718) (width 0.4) (layer F.Cu) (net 26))
 (segment (start 86.995 62.3033) (end 87.7635 63.0718) (width 0.4) (layer F.Cu) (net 26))
 (segment (start 120.528 62.3833) (end 117.465 62.3833) (width 0.4) (layer F.Cu) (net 6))
 (segment (start 125.14 57.7713) (end 120.528 62.3833) (width 0.4) (layer F.Cu) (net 6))
 (segment (start 125.14 57.34) (end 125.14 57.7713) (width 0.4) (layer F.Cu) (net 6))
 (segment (start 117.465 61.294) (end 117.465 62.3833) (width 0.4) (layer F.Cu) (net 6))
 (segment (start 117.465 54.165) (end 117.465 55.706) (width 0.4) (layer F.Cu) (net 3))
 (segment (start 116.64 53.34) (end 117.465 54.165) (width 0.4) (layer F.Cu) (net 3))
 (segment (start 95.3167 54.5167) (end 95.965 54.5167) (width 0.4) (layer F.Cu) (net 20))
 (segment (start 94.14 53.34) (end 95.3167 54.5167) (width 0.4) (layer F.Cu) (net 20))
 (segment (start 95.965 55.606) (end 95.965 54.5167) (width 0.4) (layer F.Cu) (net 20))
 (segment (start 110.4167 54.6167) (end 110.665 54.6167) (width 0.4) (layer F.Cu) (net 10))
 (segment (start 109.14 53.34) (end 110.4167 54.6167) (width 0.4) (layer F.Cu) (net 10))
 (segment (start 110.665 55.706) (end 110.665 54.6167) (width 0.4) (layer F.Cu) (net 10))
 (segment (start 118.735 53.745) (end 118.735 55.706) (width 0.4) (layer F.Cu) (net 2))
 (segment (start 119.14 53.34) (end 118.735 53.745) (width 0.4) (layer F.Cu) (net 2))
 (segment (start 98.505 53.975) (end 98.505 55.606) (width 0.4) (layer F.Cu) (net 18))
 (segment (start 99.14 53.34) (end 98.505 53.975) (width 0.4) (layer F.Cu) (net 18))
 (segment (start 102.9167 54.6167) (end 103.465 54.6167) (width 0.4) (layer F.Cu) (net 15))
 (segment (start 101.64 53.34) (end 102.9167 54.6167) (width 0.4) (layer F.Cu) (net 15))
 (segment (start 103.465 55.706) (end 103.465 54.6167) (width 0.4) (layer F.Cu) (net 15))
 (segment (start 106.005 53.975) (end 106.005 55.706) (width 0.4) (layer F.Cu) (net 13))
 (segment (start 106.64 53.34) (end 106.005 53.975) (width 0.4) (layer F.Cu) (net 13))
 (segment (start 111.6 49.3525) (end 112.7528 49.3525) (width 0.4) (layer F.Cu) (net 12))
 (segment (start 113.1003 49.7) (end 113.3475 49.7) (width 0.4) (layer F.Cu) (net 12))
 (segment (start 112.7528 49.3525) (end 113.1003 49.7) (width 0.4) (layer F.Cu) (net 12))
 (segment (start 115.3587 58.051) (end 113.205 60.2047) (width 0.4) (layer F.Cu) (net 12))
 (segment (start 115.3587 51.7112) (end 115.3587 58.051) (width 0.4) (layer F.Cu) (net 12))
 (segment (start 114.2463 50.5988) (end 115.3587 51.7112) (width 0.4) (layer F.Cu) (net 12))
 (segment (start 114.2463 49.7) (end 114.2463 50.5988) (width 0.4) (layer F.Cu) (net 12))
 (segment (start 113.3475 49.7) (end 114.2463 49.7) (width 0.4) (layer F.Cu) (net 12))
 (segment (start 113.205 61.294) (end 113.205 60.2047) (width 0.4) (layer F.Cu) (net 12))
 (segment (start 120.3633 54.6167) (end 120.005 54.6167) (width 0.4) (layer F.Cu) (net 1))
 (segment (start 121.64 53.34) (end 120.3633 54.6167) (width 0.4) (layer F.Cu) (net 1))
 (segment (start 120.005 55.706) (end 120.005 54.6167) (width 0.4) (layer F.Cu) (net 1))
 (segment (start 120.3 49.3525) (end 119.7236 49.3525) (width 0.4) (layer F.Cu) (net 7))
 (segment (start 119.4513 49.6248) (end 119.7236 49.3525) (width 0.4) (layer F.Cu) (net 7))
 (segment (start 119.4513 49.7) (end 119.4513 49.6248) (width 0.4) (layer F.Cu) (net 7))
 (segment (start 118.5525 49.7) (end 119.4513 49.7) (width 0.4) (layer F.Cu) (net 7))
 (segment (start 120.3 49.3525) (end 120.3 50.2513) (width 0.4) (layer F.Cu) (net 7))
 (segment (start 123.5253 56.8225) (end 120.005 60.3428) (width 0.4) (layer F.Cu) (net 7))
 (segment (start 123.5253 52.5641) (end 123.5253 56.8225) (width 0.4) (layer F.Cu) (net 7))
 (segment (start 121.2125 50.2513) (end 123.5253 52.5641) (width 0.4) (layer F.Cu) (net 7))
 (segment (start 120.3 50.2513) (end 121.2125 50.2513) (width 0.4) (layer F.Cu) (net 7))
 (segment (start 120.005 61.294) (end 120.005 60.3428) (width 0.4) (layer F.Cu) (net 7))
 (segment (start 111.935 53.635) (end 111.935 55.706) (width 0.4) (layer F.Cu) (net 9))
 (segment (start 111.64 53.34) (end 111.935 53.635) (width 0.4) (layer F.Cu) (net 9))
 (segment (start 104.3 49.5525) (end 103.1472 49.5525) (width 0.4) (layer F.Cu) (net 17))
 (segment (start 106.005 61.294) (end 106.005 60.2047) (width 0.4) (layer F.Cu) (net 17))
 (segment (start 102.7997 49.9) (end 103.1472 49.5525) (width 0.4) (layer F.Cu) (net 17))
 (segment (start 102.6525 49.9) (end 102.7997 49.9) (width 0.4) (layer F.Cu) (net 17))
 (segment (start 105.0764 60.2047) (end 106.005 60.2047) (width 0.4) (layer F.Cu) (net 17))
 (segment (start 100.432 55.5603) (end 105.0764 60.2047) (width 0.4) (layer F.Cu) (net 17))
 (segment (start 100.432 52.1205) (end 100.432 55.5603) (width 0.4) (layer F.Cu) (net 17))
 (segment (start 102.6525 49.9) (end 100.432 52.1205) (width 0.4) (layer F.Cu) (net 17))
 (segment (start 113.205 54.275) (end 113.205 55.706) (width 0.4) (layer F.Cu) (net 8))
 (segment (start 114.14 53.34) (end 113.205 54.275) (width 0.4) (layer F.Cu) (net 8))
 (segment (start 89.535 53.735) (end 89.535 55.626) (width 0.4) (layer F.Cu) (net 24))
 (segment (start 89.14 53.34) (end 89.535 53.735) (width 0.4) (layer F.Cu) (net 24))
 (segment (start 97.235 53.935) (end 97.235 55.606) (width 0.4) (layer F.Cu) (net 19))
 (segment (start 96.64 53.34) (end 97.235 53.935) (width 0.4) (layer F.Cu) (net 19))
 (segment (start 104.735 53.935) (end 104.735 55.706) (width 0.4) (layer F.Cu) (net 14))
 (segment (start 104.14 53.34) (end 104.735 53.935) (width 0.4) (layer F.Cu) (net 14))
 (segment (start 90.805 54.175) (end 90.805 55.626) (width 0.4) (layer F.Cu) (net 23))
 (segment (start 91.64 53.34) (end 90.805 54.175) (width 0.4) (layer F.Cu) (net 23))
 (segment (start 96.065 62.3833) (end 102.195 62.3833) (width 0.4) (layer F.Cu) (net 16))
 (segment (start 95.965 62.2833) (end 96.065 62.3833) (width 0.4) (layer F.Cu) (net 16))
 (segment (start 95.965 61.194) (end 95.965 62.2833) (width 0.4) (layer F.Cu) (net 16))
 (segment (start 102.195 61.294) (end 102.195 62.3833) (width 0.4) (layer F.Cu) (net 16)))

